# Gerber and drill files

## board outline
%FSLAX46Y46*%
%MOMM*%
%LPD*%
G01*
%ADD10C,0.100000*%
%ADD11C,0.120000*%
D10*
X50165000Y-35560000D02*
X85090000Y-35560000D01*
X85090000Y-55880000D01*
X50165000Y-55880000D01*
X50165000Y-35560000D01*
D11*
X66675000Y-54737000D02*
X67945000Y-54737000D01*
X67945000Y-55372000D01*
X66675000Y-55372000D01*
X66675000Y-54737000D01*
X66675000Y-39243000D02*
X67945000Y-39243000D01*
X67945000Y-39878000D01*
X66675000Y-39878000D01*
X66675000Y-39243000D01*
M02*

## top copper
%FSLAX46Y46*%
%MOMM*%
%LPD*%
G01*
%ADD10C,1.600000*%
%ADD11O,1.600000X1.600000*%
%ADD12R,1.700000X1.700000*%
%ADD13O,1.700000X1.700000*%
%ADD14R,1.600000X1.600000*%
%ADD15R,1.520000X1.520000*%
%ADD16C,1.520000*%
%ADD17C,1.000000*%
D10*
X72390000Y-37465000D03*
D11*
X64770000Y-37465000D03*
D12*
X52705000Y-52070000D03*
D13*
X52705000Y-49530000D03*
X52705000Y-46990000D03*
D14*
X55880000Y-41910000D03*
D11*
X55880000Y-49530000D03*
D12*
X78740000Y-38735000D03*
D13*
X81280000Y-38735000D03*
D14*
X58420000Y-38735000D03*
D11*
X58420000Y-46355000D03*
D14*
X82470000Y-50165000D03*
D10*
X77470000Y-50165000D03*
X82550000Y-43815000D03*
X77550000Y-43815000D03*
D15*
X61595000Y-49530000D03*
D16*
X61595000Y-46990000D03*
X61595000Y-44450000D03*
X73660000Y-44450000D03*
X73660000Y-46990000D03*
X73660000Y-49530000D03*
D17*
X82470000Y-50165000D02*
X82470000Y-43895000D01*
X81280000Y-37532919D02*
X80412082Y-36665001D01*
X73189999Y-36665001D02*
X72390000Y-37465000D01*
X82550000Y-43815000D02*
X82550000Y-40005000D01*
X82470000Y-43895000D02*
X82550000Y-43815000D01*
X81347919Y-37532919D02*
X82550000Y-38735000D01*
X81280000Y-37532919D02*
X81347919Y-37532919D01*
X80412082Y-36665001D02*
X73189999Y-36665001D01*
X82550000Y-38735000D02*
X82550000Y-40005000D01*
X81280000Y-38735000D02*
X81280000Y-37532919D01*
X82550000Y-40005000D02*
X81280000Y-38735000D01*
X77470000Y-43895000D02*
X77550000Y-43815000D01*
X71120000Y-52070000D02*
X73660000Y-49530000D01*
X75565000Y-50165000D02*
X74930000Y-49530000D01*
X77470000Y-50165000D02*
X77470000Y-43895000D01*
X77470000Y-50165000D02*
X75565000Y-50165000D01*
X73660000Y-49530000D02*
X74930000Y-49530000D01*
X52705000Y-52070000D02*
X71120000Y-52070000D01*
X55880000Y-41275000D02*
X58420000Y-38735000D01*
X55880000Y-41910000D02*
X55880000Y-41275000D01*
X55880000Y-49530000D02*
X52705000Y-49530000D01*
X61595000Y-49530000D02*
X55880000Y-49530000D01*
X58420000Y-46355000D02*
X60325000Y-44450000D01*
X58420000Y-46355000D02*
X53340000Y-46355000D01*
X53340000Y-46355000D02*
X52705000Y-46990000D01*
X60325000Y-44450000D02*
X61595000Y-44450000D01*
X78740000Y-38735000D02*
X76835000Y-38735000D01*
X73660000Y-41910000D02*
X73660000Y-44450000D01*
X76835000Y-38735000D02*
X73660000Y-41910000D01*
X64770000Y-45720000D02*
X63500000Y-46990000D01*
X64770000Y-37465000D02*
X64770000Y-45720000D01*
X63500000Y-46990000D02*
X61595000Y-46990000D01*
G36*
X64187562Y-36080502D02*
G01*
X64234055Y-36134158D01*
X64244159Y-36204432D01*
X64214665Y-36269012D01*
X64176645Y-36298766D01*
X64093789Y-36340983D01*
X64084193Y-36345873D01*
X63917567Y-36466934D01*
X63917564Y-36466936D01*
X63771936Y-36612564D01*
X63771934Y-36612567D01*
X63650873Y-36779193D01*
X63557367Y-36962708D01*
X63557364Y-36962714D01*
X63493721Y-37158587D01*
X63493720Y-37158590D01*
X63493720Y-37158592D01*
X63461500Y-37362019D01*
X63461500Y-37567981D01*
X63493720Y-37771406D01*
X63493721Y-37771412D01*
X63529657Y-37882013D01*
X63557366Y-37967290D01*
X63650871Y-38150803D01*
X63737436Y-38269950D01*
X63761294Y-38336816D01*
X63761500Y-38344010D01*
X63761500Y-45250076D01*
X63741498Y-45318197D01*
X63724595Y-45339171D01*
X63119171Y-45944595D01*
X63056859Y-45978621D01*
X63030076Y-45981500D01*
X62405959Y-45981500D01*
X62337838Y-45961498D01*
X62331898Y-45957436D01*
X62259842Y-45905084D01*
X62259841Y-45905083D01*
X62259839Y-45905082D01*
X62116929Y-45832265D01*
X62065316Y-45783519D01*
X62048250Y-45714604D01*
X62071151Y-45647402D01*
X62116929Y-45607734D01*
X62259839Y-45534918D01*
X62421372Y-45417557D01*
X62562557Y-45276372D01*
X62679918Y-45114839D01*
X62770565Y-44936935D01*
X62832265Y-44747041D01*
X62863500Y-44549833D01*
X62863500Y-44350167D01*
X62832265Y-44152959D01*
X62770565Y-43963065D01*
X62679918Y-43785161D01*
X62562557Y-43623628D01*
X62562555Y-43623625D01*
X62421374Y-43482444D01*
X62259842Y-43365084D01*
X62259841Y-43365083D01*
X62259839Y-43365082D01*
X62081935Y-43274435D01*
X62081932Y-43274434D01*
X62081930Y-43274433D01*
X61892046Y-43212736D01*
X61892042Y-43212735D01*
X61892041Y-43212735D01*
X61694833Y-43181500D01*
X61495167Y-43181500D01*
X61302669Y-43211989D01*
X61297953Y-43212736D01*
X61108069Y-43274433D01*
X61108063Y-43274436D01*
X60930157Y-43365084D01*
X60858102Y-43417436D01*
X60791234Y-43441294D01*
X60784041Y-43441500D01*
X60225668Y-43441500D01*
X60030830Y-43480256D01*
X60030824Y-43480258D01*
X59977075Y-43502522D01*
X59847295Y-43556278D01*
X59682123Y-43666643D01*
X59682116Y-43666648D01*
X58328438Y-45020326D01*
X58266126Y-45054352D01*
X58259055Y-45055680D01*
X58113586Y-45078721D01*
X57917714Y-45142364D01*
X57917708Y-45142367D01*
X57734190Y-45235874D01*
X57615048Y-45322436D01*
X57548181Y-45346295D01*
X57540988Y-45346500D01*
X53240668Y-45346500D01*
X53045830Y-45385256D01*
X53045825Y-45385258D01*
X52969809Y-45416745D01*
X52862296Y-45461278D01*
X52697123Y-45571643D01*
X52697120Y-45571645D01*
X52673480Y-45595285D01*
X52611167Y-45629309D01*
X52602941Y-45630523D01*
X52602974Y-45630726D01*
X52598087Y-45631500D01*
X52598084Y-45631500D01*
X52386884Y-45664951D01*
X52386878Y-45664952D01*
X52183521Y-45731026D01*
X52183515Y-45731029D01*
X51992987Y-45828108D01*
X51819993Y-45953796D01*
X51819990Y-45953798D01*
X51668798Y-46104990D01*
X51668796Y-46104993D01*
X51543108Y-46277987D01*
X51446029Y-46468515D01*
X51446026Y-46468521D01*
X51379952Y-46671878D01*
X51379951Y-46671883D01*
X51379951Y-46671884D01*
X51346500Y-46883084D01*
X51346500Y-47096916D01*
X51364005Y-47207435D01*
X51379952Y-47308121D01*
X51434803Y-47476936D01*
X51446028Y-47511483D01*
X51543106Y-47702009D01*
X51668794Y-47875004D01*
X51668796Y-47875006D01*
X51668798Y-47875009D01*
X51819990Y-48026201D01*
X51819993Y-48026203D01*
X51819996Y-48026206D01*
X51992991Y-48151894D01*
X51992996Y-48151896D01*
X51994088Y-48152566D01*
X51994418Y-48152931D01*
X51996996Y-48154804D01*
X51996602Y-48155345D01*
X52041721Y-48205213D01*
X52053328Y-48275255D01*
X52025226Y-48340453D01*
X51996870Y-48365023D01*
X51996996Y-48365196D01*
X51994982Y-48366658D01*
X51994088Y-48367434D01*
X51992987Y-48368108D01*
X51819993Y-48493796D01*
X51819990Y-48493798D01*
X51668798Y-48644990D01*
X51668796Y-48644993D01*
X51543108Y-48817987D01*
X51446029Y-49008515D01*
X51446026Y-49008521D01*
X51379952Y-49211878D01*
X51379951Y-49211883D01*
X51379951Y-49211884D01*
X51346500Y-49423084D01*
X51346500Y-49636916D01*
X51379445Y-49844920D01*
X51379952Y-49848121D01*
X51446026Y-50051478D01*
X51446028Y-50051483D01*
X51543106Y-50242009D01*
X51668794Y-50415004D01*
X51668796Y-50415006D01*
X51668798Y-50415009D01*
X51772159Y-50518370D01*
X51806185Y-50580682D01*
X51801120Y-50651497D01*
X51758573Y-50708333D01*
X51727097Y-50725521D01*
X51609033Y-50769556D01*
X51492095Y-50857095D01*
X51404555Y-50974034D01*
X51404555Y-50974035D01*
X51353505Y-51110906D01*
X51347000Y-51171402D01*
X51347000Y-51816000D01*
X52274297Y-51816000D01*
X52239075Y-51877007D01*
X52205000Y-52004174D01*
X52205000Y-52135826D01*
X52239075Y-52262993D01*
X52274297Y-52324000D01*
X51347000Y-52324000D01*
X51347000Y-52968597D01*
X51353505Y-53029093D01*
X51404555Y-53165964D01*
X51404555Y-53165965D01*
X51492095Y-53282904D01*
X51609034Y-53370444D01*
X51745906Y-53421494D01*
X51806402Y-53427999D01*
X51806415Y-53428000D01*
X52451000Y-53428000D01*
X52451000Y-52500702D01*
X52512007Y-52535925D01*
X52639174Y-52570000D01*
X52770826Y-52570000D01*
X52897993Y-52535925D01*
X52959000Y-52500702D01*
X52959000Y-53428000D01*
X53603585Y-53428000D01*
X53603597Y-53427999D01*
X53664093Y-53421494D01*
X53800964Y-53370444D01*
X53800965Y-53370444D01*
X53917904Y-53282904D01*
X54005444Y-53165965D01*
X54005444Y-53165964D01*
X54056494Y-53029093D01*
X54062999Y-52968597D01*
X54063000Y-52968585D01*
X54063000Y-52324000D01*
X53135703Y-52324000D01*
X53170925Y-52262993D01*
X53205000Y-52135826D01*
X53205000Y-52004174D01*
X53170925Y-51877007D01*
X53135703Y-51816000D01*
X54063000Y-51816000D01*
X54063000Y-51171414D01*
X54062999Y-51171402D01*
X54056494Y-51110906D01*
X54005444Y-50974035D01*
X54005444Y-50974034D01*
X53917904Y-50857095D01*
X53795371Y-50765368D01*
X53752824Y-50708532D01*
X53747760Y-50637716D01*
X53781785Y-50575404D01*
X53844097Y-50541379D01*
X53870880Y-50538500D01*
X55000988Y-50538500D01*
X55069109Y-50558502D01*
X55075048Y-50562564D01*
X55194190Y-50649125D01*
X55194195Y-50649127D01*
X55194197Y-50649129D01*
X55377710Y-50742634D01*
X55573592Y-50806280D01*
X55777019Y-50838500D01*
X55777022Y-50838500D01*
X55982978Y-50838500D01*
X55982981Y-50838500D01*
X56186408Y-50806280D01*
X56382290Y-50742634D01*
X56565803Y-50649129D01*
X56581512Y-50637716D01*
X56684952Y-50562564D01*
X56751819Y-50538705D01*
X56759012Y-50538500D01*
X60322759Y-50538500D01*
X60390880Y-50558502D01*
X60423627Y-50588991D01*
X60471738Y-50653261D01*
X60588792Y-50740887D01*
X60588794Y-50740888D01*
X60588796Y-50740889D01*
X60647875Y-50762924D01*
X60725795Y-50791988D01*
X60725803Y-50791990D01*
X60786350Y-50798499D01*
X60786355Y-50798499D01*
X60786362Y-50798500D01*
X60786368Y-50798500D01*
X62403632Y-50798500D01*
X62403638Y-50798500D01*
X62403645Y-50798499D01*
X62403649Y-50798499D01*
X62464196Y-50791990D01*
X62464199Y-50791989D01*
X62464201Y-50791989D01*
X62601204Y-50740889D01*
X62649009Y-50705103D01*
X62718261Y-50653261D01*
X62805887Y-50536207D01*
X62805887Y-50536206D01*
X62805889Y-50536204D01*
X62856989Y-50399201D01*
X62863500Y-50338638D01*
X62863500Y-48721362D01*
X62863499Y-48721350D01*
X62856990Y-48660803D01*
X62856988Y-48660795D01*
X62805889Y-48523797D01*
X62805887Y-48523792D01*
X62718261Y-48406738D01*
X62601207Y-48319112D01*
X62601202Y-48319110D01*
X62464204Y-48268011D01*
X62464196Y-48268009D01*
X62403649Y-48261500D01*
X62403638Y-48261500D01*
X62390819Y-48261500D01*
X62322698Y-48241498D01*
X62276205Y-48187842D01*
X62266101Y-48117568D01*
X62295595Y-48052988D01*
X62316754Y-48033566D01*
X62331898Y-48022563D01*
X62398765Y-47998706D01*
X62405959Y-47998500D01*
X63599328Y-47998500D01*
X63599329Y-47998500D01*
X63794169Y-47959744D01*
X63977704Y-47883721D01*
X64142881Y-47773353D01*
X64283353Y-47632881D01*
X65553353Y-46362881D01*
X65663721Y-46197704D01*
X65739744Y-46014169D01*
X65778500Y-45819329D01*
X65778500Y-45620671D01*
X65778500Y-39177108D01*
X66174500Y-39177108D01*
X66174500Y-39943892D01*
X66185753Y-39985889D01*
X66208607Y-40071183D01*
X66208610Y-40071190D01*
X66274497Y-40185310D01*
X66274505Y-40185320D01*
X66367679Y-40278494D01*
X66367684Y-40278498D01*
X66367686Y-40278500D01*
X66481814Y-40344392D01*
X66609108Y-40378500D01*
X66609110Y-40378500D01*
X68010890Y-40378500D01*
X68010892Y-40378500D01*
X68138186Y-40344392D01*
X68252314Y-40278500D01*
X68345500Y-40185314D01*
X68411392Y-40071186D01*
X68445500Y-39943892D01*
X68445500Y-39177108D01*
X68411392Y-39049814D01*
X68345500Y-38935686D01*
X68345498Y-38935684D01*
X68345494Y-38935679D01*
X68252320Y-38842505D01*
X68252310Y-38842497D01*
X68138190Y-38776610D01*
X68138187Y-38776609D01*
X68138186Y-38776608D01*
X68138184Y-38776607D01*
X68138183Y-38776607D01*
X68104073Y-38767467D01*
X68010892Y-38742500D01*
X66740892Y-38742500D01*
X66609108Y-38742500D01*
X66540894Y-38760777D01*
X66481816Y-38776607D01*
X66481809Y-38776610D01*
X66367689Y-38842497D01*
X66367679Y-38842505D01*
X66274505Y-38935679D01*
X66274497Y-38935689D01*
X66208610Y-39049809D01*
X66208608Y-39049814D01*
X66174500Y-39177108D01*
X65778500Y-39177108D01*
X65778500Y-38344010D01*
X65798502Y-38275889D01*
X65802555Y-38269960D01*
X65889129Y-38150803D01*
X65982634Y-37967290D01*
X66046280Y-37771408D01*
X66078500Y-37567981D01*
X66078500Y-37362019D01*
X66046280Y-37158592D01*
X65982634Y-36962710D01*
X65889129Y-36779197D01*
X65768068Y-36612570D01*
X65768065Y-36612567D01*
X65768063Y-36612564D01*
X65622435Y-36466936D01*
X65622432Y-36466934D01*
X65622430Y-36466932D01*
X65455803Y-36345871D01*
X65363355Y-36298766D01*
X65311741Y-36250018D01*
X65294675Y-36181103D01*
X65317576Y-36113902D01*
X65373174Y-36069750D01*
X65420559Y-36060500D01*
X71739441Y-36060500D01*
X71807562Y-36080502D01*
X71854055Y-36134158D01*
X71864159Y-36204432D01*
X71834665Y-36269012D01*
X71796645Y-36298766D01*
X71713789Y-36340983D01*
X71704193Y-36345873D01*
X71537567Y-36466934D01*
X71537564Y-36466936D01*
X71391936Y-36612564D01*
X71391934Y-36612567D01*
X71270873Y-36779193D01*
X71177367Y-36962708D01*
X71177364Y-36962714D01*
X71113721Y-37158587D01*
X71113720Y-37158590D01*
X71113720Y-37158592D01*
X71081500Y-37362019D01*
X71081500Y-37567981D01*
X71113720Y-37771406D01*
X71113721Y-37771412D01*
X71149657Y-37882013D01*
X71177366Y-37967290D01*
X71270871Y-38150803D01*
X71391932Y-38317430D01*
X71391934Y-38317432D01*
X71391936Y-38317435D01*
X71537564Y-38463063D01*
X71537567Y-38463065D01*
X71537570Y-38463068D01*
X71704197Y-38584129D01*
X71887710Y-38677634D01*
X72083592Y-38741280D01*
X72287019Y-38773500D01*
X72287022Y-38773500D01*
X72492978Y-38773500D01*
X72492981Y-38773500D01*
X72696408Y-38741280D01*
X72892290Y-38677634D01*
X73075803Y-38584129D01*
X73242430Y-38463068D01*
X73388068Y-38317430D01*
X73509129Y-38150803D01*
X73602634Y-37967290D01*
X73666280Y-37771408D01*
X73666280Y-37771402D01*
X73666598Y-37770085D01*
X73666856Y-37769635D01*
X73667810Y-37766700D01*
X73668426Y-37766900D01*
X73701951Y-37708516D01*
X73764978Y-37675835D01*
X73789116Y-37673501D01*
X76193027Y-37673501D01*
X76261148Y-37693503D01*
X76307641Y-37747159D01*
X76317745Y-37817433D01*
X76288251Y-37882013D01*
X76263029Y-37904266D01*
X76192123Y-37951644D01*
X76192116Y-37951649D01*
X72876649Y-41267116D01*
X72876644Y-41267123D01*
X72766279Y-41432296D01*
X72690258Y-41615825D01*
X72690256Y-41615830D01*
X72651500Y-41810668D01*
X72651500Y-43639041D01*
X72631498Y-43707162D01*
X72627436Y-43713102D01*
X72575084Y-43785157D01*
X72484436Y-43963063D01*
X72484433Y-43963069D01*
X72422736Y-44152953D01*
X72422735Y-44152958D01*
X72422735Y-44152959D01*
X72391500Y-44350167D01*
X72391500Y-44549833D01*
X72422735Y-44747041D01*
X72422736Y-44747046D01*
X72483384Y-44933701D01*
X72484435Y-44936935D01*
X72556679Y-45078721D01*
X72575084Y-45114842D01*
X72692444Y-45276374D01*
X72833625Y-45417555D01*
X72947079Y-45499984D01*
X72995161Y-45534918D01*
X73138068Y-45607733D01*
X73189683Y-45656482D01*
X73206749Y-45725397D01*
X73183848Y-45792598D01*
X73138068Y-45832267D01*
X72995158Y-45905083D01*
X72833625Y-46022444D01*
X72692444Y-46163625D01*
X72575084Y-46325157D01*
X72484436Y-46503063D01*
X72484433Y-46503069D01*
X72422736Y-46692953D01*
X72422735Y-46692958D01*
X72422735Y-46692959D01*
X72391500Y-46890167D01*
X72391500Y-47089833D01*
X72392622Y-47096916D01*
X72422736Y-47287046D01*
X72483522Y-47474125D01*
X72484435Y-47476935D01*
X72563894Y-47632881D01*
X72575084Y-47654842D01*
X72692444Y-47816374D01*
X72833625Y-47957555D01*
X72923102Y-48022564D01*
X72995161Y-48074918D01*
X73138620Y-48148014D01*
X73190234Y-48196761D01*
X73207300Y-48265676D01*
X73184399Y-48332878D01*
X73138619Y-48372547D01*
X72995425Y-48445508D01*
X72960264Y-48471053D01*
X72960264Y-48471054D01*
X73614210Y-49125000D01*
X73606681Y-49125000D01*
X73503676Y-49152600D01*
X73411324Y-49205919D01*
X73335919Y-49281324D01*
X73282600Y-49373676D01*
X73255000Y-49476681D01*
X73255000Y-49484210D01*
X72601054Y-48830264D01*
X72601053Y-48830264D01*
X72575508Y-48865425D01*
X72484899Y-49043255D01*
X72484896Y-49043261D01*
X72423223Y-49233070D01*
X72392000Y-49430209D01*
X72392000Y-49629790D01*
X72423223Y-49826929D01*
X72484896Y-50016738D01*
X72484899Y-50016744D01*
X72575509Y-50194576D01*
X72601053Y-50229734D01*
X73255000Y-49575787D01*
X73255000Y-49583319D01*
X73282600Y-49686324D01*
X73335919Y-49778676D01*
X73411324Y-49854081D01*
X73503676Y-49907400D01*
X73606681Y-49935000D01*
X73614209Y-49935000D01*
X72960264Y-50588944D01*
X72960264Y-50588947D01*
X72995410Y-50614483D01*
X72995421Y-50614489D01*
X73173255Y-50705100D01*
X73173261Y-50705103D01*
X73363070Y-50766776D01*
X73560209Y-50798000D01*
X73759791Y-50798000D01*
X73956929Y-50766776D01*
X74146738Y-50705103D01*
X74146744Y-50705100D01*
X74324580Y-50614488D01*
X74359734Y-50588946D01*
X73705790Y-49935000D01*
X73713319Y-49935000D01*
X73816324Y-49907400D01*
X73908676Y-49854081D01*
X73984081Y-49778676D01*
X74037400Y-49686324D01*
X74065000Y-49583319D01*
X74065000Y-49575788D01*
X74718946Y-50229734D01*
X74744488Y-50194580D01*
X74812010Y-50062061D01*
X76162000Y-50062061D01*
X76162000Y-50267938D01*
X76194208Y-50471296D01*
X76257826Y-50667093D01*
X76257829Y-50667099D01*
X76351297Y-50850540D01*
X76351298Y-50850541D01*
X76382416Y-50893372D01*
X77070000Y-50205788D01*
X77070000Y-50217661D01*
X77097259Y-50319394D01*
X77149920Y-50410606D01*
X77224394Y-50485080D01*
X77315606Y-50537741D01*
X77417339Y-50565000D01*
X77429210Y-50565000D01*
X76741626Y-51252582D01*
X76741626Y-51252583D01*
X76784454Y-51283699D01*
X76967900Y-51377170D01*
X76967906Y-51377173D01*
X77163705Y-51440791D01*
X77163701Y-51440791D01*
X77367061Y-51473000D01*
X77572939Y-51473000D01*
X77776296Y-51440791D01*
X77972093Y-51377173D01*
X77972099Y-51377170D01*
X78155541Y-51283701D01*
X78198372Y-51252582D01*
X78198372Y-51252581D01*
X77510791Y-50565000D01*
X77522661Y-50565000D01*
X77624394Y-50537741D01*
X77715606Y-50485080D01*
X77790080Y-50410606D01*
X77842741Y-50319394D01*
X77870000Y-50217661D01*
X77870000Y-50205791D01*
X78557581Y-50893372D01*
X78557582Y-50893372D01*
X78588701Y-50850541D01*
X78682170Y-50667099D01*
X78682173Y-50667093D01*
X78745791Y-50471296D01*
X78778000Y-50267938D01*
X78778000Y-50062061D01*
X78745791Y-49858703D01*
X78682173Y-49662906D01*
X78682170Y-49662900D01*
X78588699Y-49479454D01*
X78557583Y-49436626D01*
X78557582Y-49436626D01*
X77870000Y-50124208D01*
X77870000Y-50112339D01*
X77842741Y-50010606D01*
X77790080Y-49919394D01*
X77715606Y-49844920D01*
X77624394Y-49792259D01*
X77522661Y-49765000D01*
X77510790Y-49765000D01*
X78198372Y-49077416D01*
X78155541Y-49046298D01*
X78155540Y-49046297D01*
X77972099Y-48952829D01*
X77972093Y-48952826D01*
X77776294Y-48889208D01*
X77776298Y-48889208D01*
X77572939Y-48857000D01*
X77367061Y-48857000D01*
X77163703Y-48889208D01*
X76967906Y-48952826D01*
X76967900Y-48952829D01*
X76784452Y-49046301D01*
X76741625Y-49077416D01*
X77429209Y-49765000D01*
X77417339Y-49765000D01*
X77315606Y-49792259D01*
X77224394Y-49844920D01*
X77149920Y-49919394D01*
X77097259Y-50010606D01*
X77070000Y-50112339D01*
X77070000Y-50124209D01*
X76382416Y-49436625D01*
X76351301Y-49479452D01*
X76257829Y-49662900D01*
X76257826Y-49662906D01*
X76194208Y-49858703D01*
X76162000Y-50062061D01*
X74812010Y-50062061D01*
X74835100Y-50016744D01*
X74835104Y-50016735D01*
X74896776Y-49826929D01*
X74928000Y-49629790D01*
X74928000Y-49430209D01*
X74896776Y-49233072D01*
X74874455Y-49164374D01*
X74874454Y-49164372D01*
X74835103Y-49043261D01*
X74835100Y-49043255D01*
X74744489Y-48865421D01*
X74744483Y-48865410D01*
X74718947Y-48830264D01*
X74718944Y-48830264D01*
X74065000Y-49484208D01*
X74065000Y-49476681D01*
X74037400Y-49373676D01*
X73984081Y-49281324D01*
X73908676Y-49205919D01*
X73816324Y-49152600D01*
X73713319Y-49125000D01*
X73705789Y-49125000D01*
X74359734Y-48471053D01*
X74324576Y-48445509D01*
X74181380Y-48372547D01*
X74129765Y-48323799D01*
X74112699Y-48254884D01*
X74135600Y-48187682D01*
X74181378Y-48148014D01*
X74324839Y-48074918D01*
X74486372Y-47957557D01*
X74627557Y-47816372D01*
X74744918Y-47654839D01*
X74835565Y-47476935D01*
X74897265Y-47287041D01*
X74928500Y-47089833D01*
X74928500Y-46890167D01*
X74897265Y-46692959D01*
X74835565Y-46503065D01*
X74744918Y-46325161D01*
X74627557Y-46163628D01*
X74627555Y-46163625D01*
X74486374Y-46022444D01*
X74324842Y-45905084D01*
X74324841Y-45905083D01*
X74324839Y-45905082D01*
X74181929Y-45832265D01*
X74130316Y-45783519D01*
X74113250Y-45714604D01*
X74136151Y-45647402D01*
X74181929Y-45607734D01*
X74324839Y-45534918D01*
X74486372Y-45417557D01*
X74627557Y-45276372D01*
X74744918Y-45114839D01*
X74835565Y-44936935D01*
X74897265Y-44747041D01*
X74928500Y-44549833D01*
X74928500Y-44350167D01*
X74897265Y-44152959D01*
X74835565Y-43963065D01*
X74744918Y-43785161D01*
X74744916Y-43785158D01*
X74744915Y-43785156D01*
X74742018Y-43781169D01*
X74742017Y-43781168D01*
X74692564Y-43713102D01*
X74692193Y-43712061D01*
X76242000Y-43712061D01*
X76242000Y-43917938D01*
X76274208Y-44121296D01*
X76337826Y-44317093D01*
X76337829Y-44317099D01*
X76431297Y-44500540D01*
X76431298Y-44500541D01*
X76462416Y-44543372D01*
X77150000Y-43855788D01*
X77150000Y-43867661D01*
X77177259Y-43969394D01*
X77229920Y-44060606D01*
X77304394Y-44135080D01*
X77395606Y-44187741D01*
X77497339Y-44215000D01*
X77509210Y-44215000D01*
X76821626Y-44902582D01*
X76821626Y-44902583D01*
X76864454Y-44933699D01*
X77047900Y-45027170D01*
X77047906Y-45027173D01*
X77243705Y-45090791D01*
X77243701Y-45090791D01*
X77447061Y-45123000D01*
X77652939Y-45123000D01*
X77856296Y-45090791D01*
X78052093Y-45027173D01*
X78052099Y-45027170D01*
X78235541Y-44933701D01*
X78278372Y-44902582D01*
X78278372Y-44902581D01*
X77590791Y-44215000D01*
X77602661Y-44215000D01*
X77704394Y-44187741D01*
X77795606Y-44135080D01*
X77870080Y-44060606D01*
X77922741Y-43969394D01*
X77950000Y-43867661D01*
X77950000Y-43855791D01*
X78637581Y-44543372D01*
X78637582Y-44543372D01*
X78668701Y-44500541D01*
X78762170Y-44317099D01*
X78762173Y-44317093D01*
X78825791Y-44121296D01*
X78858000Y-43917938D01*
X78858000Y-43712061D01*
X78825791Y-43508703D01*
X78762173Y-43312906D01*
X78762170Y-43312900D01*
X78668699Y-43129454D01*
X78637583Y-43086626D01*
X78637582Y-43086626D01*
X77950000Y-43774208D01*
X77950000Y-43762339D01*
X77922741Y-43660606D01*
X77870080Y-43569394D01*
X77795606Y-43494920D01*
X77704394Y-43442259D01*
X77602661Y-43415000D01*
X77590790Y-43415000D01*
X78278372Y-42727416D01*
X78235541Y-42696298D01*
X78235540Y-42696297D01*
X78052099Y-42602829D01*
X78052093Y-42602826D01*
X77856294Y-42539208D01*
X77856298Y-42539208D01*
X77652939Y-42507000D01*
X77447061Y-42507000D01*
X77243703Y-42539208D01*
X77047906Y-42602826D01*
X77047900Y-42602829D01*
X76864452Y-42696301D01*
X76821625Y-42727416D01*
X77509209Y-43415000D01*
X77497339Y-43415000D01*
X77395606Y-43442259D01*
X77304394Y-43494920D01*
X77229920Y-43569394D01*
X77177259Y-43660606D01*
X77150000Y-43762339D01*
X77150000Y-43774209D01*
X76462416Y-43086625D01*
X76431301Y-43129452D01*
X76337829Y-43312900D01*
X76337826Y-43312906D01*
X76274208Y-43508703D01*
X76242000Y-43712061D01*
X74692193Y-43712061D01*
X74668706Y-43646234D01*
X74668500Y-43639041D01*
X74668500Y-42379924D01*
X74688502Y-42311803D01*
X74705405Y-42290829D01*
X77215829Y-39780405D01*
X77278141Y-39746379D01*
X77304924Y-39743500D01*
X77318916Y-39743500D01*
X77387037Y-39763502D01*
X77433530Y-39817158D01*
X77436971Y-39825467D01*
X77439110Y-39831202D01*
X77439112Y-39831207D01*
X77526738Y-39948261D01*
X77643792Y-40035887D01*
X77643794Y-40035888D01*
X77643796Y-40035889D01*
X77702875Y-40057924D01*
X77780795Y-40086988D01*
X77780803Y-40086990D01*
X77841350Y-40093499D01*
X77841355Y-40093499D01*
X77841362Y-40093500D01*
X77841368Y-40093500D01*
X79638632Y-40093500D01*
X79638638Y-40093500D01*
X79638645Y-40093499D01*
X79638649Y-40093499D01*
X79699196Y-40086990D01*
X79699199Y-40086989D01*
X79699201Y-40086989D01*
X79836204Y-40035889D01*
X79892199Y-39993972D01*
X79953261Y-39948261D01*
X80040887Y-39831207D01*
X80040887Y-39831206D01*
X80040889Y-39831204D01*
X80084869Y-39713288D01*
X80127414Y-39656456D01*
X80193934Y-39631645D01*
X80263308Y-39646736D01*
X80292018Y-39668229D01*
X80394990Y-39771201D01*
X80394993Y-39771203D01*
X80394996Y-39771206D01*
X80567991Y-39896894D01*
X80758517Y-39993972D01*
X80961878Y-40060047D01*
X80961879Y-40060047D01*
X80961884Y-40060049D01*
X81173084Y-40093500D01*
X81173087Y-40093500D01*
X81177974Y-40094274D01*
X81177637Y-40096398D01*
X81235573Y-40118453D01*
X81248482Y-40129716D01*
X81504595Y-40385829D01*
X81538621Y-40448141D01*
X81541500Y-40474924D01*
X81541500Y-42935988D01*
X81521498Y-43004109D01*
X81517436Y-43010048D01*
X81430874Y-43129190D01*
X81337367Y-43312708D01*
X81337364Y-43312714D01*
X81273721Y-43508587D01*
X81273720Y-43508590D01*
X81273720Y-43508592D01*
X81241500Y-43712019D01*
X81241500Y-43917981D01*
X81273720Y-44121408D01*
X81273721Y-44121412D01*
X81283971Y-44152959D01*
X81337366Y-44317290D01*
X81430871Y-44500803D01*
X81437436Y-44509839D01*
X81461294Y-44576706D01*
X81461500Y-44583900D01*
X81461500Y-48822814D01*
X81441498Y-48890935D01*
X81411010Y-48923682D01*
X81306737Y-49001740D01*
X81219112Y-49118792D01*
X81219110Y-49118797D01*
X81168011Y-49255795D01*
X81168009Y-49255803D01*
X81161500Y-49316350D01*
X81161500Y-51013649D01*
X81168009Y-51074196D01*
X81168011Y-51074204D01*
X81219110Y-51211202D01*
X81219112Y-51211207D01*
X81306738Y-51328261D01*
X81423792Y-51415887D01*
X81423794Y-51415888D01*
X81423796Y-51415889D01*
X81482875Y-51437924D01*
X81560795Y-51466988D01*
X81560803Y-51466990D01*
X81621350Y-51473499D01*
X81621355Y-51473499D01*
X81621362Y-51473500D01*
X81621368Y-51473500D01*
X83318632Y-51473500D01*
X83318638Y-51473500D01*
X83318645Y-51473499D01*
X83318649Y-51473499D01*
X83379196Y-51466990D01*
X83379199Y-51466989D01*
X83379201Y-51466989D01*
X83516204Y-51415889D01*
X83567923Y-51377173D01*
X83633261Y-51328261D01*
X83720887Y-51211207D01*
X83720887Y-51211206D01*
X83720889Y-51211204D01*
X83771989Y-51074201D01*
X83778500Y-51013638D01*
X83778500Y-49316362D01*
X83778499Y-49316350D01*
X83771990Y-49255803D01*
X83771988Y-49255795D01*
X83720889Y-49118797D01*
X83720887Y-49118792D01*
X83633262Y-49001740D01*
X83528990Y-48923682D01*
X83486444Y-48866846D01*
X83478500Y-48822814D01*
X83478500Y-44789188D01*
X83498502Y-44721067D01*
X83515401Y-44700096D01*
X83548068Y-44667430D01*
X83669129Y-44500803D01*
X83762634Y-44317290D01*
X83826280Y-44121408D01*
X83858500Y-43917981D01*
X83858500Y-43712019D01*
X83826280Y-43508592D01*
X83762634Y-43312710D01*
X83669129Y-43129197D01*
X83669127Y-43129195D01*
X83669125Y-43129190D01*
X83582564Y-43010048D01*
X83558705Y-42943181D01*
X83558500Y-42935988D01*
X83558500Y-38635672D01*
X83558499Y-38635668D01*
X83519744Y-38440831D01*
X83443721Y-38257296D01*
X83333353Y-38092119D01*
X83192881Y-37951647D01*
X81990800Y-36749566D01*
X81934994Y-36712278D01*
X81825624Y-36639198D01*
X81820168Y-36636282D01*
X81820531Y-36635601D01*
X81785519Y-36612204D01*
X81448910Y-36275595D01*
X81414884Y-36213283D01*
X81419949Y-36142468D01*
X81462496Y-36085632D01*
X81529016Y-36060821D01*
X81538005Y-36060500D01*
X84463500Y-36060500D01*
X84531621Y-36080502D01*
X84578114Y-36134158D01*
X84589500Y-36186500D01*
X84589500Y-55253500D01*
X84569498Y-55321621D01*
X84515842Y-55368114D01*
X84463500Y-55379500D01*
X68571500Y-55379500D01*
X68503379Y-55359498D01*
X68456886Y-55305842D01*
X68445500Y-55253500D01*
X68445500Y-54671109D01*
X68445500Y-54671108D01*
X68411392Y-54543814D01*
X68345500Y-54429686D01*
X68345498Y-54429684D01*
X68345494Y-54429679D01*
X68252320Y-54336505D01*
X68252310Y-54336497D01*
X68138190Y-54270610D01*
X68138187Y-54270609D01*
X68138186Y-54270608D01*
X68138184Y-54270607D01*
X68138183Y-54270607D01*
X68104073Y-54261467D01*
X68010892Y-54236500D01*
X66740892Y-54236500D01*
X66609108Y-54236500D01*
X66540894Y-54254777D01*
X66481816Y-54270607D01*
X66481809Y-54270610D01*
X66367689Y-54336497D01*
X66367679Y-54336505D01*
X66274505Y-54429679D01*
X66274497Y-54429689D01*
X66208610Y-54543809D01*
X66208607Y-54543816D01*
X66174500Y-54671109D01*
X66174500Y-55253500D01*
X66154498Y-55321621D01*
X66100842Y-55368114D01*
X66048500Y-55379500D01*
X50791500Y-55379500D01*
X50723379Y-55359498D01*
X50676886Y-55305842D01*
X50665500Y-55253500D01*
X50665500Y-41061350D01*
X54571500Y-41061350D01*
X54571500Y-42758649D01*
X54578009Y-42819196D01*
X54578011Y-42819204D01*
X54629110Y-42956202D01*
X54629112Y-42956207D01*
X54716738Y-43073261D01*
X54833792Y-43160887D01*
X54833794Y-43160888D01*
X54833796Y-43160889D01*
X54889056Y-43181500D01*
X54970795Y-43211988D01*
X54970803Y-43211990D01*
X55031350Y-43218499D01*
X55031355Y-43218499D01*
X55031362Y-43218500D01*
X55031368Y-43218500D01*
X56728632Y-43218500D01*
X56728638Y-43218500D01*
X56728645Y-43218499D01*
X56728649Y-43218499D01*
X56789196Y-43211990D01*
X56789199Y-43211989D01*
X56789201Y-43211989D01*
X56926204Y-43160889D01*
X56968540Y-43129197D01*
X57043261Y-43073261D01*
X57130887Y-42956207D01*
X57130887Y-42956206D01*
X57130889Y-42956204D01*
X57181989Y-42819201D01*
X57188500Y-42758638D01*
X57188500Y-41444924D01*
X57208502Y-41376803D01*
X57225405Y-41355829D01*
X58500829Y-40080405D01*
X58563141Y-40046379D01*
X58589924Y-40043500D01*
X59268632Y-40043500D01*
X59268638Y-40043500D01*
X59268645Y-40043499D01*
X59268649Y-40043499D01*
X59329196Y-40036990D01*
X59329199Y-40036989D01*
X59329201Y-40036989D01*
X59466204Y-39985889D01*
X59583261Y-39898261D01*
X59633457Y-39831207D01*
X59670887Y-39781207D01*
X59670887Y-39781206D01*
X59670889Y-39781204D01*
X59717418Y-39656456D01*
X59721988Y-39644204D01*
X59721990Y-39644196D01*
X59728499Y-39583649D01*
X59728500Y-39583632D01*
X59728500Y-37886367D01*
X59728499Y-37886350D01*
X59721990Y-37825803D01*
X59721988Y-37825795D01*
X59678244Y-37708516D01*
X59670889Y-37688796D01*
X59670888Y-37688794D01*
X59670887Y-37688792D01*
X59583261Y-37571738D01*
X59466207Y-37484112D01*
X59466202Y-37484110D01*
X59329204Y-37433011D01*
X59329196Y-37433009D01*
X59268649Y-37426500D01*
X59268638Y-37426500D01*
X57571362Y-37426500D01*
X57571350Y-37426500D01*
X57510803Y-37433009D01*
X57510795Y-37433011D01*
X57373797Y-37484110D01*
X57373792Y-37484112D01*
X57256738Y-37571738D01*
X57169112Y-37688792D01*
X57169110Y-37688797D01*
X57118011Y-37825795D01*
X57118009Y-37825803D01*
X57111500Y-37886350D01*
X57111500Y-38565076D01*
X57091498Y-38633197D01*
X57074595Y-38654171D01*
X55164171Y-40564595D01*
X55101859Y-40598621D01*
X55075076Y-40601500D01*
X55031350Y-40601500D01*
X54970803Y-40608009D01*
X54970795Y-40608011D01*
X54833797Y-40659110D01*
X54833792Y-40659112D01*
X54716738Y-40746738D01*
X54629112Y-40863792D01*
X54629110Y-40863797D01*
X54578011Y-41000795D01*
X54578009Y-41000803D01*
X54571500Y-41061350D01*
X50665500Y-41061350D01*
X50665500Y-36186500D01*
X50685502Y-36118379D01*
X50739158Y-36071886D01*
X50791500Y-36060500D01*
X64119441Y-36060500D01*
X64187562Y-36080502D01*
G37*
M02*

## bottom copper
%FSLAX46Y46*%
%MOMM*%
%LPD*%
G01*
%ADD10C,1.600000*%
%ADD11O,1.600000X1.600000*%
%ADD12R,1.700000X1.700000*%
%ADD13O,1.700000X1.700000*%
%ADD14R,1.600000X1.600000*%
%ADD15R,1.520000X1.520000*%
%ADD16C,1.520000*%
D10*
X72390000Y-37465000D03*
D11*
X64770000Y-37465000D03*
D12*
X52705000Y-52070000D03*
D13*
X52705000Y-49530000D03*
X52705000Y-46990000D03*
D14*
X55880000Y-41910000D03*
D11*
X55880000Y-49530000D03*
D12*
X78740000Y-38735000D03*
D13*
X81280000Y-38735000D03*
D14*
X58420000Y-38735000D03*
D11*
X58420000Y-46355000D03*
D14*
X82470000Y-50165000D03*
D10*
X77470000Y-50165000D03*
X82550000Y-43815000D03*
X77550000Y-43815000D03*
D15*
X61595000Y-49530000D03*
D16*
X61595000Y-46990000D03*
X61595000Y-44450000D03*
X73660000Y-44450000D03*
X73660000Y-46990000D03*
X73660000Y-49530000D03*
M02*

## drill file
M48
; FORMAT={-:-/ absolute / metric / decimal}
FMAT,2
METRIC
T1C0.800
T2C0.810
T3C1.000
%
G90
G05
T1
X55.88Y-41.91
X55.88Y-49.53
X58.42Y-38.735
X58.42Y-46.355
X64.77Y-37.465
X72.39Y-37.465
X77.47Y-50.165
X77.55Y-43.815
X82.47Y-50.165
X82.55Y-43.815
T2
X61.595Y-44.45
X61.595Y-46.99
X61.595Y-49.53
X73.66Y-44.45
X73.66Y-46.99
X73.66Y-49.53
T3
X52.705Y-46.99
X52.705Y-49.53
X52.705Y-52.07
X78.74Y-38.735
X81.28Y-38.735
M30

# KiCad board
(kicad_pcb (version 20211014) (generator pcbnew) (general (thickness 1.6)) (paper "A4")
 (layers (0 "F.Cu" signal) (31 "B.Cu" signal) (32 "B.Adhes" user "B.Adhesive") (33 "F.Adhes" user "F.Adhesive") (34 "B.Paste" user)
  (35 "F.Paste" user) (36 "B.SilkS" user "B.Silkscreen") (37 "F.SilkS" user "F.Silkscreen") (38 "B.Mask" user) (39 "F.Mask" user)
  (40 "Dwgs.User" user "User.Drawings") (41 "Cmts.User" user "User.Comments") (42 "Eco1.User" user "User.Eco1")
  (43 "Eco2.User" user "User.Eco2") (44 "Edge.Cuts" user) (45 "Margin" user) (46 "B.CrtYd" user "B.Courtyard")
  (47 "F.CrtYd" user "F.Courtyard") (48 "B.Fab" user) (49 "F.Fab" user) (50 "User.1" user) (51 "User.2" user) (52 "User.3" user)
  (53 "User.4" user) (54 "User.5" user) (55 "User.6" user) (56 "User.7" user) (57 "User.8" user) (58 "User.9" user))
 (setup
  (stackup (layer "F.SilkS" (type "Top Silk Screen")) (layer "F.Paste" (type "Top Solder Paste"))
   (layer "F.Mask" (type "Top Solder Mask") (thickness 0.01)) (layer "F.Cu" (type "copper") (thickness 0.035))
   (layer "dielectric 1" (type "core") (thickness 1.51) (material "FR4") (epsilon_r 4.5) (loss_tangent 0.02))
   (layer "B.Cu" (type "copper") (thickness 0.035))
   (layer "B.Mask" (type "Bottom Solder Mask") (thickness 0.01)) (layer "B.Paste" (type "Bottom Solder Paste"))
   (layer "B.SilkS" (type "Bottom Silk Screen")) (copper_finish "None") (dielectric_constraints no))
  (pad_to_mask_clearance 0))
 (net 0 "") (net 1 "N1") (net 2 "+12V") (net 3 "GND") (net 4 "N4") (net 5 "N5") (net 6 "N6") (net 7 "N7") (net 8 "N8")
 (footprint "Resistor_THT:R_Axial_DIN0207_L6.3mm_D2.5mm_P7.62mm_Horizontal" (layer "F.Cu") (at 72.39 37.465 180)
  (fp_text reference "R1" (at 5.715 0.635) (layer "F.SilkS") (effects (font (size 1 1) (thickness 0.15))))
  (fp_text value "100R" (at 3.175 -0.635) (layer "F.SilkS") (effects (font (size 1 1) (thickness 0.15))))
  (pad "1" thru_hole circle (at 0 0 180) (size 1.6 1.6) (drill 0.8) (layers *.Cu *.Mask) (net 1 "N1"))
  (pad "2" thru_hole oval (at 7.62 0 180) (size 1.6 1.6) (drill 0.8) (layers *.Cu *.Mask) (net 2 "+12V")))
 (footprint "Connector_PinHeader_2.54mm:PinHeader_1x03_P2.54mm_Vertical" (layer "F.Cu") (at 52.705 52.07 180)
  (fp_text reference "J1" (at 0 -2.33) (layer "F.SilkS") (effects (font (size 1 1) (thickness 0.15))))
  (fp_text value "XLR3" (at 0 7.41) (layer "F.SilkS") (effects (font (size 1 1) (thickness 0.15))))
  (pad "1" thru_hole rect (at 0 0 180) (size 1.7 1.7) (drill 1) (layers *.Cu *.Mask) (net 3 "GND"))
  (pad "2" thru_hole oval (at 0 2.54 180) (size 1.7 1.7) (drill 1) (layers *.Cu *.Mask) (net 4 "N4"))
  (pad "3" thru_hole oval (at 0 5.08 180) (size 1.7 1.7) (drill 1) (layers *.Cu *.Mask) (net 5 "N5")))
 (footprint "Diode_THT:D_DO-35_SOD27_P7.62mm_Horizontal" (layer "F.Cu") (at 55.88 41.91 -90)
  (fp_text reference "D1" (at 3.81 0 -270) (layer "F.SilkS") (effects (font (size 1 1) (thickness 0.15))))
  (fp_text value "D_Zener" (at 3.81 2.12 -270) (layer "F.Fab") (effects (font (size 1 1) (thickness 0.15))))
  (pad "1" thru_hole rect (at 0 0 270) (size 1.6 1.6) (drill 0.8) (layers *.Cu *.Mask) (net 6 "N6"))
  (pad "2" thru_hole oval (at 7.62 0 270) (size 1.6 1.6) (drill 0.8) (layers *.Cu *.Mask) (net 4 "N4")))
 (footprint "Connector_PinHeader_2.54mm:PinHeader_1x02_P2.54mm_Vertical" (layer "F.Cu") (at 78.74 38.735 90)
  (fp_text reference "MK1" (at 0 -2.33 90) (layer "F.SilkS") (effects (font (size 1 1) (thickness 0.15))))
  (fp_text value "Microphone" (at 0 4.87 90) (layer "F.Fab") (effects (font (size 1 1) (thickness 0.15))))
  (pad "1" thru_hole rect (at 0 0 90) (size 1.7 1.7) (drill 1) (layers *.Cu *.Mask) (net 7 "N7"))
  (pad "2" thru_hole oval (at 0 2.54 90) (size 1.7 1.7) (drill 1) (layers *.Cu *.Mask) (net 1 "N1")))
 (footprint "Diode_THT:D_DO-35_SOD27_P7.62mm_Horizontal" (layer "F.Cu") (at 58.42 38.735 -90)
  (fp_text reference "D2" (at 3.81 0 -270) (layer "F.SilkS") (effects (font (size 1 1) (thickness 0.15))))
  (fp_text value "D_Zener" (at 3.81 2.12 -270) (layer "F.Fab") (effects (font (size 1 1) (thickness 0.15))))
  (pad "1" thru_hole rect (at 0 0 270) (size 1.6 1.6) (drill 0.8) (layers *.Cu *.Mask) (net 6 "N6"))
  (pad "2" thru_hole oval (at 7.62 0 270) (size 1.6 1.6) (drill 0.8) (layers *.Cu *.Mask) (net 5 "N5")))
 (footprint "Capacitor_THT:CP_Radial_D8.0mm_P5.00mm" (layer "F.Cu") (at 82.47 50.165 180)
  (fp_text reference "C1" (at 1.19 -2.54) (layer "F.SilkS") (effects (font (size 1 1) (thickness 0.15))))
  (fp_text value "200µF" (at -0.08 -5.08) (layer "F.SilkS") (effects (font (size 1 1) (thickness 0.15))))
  (pad "1" thru_hole rect (at 0 0 180) (size 1.6 1.6) (drill 0.8) (layers *.Cu *.Mask) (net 1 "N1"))
  (pad "2" thru_hole circle (at 5 0 180) (size 1.6 1.6) (drill 0.8) (layers *.Cu *.Mask) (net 3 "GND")))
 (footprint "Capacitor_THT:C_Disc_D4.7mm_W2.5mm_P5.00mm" (layer "F.Cu") (at 82.55 43.815 180)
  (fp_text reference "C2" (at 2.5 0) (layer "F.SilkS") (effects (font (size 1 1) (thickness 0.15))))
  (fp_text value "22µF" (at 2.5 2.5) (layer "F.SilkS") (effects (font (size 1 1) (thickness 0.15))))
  (pad "1" thru_hole circle (at 0 0 180) (size 1.6 1.6) (drill 0.8) (layers *.Cu *.Mask) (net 1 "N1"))
  (pad "2" thru_hole circle (at 5 0 180) (size 1.6 1.6) (drill 0.8) (layers *.Cu *.Mask) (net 3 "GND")))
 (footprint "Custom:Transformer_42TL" (layer "B.Cu") (at 72.39 52.07)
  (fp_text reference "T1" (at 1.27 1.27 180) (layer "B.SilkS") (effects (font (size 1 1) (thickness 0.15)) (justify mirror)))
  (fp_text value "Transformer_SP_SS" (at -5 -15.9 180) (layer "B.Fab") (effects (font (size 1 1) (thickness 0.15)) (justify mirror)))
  (fp_rect (start -5.715 3.302) (end -4.445 2.667) (layer "Edge.Cuts") (width 0.12) (fill none))
  (fp_rect (start -5.715 -12.192) (end -4.445 -12.827) (layer "Edge.Cuts") (width 0.12) (fill none))
  (pad "1" thru_hole rect (at -10.795 -2.54) (size 1.52 1.52) (drill 0.81) (layers *.Cu *.Mask) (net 4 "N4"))
  (pad "2" thru_hole circle (at -10.795 -5.08) (size 1.52 1.52) (drill 0.81) (layers *.Cu *.Mask) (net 2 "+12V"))
  (pad "3" thru_hole circle (at -10.795 -7.62) (size 1.52 1.52) (drill 0.81) (layers *.Cu *.Mask) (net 5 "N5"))
  (pad "4" thru_hole circle (at 1.27 -7.62) (size 1.52 1.52) (drill 0.81) (layers *.Cu *.Mask) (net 7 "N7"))
  (pad "5" thru_hole circle (at 1.27 -5.08) (size 1.52 1.52) (drill 0.81) (layers *.Cu *.Mask) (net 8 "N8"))
  (pad "6" thru_hole circle (at 1.27 -2.54) (size 1.52 1.52) (drill 0.81) (layers *.Cu *.Mask) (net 3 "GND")))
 (gr_rect (start 50.165 35.56) (end 85.09 55.88) (layer "Edge.Cuts") (width 0.1) (fill none))
 (segment (start 82.47 50.165) (end 82.47 43.895) (width 1) (layer "F.Cu") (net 1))
 (segment (start 81.28 37.532919) (end 80.412082 36.665001) (width 1) (layer "F.Cu") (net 1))
 (segment (start 73.189999 36.665001) (end 72.39 37.465) (width 1) (layer "F.Cu") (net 1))
 (segment (start 82.55 43.815) (end 82.55 40.005) (width 1) (layer "F.Cu") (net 1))
 (segment (start 82.47 43.895) (end 82.55 43.815) (width 1) (layer "F.Cu") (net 1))
 (segment (start 81.347919 37.532919) (end 82.55 38.735) (width 1) (layer "F.Cu") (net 1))
 (segment (start 81.28 37.532919) (end 81.347919 37.532919) (width 1) (layer "F.Cu") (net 1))
 (segment (start 80.412082 36.665001) (end 73.189999 36.665001) (width 1) (layer "F.Cu") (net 1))
 (segment (start 82.55 38.735) (end 82.55 40.005) (width 1) (layer "F.Cu") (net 1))
 (segment (start 81.28 38.735) (end 81.28 37.532919) (width 1) (layer "F.Cu") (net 1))
 (segment (start 82.55 40.005) (end 81.28 38.735) (width 1) (layer "F.Cu") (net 1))
 (segment (start 77.47 43.895) (end 77.55 43.815) (width 1) (layer "F.Cu") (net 3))
 (segment (start 71.12 52.07) (end 73.66 49.53) (width 1) (layer "F.Cu") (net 3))
 (segment (start 75.565 50.165) (end 74.93 49.53) (width 1) (layer "F.Cu") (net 3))
 (segment (start 77.47 50.165) (end 77.47 43.895) (width 1) (layer "F.Cu") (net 3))
 (segment (start 77.47 50.165) (end 75.565 50.165) (width 1) (layer "F.Cu") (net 3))
 (segment (start 73.66 49.53) (end 74.93 49.53) (width 1) (layer "F.Cu") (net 3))
 (segment (start 52.705 52.07) (end 71.12 52.07) (width 1) (layer "F.Cu") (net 3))
 (segment (start 55.88 41.275) (end 58.42 38.735) (width 1) (layer "F.Cu") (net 6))
 (segment (start 55.88 41.91) (end 55.88 41.275) (width 1) (layer "F.Cu") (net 6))
 (segment (start 55.88 49.53) (end 52.705 49.53) (width 1) (layer "F.Cu") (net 4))
 (segment (start 61.595 49.53) (end 55.88 49.53) (width 1) (layer "F.Cu") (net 4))
 (segment (start 58.42 46.355) (end 60.325 44.45) (width 1) (layer "F.Cu") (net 5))
 (segment (start 58.42 46.355) (end 53.34 46.355) (width 1) (layer "F.Cu") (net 5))
 (segment (start 53.34 46.355) (end 52.705 46.99) (width 1) (layer "F.Cu") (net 5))
 (segment (start 60.325 44.45) (end 61.595 44.45) (width 1) (layer "F.Cu") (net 5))
 (segment (start 78.74 38.735) (end 76.835 38.735) (width 1) (layer "F.Cu") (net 7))
 (segment (start 73.66 41.91) (end 73.66 44.45) (width 1) (layer "F.Cu") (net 7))
 (segment (start 76.835 38.735) (end 73.66 41.91) (width 1) (layer "F.Cu") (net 7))
 (segment (start 64.77 45.72) (end 63.5 46.99) (width 1) (layer "F.Cu") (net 2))
 (segment (start 64.77 37.465) (end 64.77 45.72) (width 1) (layer "F.Cu") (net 2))
 (segment (start 63.5 46.99) (end 61.595 46.99) (width 1) (layer "F.Cu") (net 2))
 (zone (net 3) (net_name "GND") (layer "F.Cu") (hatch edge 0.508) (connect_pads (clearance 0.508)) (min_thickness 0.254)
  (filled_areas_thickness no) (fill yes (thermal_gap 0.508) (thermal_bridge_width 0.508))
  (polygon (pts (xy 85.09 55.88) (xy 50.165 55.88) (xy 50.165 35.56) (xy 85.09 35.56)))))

